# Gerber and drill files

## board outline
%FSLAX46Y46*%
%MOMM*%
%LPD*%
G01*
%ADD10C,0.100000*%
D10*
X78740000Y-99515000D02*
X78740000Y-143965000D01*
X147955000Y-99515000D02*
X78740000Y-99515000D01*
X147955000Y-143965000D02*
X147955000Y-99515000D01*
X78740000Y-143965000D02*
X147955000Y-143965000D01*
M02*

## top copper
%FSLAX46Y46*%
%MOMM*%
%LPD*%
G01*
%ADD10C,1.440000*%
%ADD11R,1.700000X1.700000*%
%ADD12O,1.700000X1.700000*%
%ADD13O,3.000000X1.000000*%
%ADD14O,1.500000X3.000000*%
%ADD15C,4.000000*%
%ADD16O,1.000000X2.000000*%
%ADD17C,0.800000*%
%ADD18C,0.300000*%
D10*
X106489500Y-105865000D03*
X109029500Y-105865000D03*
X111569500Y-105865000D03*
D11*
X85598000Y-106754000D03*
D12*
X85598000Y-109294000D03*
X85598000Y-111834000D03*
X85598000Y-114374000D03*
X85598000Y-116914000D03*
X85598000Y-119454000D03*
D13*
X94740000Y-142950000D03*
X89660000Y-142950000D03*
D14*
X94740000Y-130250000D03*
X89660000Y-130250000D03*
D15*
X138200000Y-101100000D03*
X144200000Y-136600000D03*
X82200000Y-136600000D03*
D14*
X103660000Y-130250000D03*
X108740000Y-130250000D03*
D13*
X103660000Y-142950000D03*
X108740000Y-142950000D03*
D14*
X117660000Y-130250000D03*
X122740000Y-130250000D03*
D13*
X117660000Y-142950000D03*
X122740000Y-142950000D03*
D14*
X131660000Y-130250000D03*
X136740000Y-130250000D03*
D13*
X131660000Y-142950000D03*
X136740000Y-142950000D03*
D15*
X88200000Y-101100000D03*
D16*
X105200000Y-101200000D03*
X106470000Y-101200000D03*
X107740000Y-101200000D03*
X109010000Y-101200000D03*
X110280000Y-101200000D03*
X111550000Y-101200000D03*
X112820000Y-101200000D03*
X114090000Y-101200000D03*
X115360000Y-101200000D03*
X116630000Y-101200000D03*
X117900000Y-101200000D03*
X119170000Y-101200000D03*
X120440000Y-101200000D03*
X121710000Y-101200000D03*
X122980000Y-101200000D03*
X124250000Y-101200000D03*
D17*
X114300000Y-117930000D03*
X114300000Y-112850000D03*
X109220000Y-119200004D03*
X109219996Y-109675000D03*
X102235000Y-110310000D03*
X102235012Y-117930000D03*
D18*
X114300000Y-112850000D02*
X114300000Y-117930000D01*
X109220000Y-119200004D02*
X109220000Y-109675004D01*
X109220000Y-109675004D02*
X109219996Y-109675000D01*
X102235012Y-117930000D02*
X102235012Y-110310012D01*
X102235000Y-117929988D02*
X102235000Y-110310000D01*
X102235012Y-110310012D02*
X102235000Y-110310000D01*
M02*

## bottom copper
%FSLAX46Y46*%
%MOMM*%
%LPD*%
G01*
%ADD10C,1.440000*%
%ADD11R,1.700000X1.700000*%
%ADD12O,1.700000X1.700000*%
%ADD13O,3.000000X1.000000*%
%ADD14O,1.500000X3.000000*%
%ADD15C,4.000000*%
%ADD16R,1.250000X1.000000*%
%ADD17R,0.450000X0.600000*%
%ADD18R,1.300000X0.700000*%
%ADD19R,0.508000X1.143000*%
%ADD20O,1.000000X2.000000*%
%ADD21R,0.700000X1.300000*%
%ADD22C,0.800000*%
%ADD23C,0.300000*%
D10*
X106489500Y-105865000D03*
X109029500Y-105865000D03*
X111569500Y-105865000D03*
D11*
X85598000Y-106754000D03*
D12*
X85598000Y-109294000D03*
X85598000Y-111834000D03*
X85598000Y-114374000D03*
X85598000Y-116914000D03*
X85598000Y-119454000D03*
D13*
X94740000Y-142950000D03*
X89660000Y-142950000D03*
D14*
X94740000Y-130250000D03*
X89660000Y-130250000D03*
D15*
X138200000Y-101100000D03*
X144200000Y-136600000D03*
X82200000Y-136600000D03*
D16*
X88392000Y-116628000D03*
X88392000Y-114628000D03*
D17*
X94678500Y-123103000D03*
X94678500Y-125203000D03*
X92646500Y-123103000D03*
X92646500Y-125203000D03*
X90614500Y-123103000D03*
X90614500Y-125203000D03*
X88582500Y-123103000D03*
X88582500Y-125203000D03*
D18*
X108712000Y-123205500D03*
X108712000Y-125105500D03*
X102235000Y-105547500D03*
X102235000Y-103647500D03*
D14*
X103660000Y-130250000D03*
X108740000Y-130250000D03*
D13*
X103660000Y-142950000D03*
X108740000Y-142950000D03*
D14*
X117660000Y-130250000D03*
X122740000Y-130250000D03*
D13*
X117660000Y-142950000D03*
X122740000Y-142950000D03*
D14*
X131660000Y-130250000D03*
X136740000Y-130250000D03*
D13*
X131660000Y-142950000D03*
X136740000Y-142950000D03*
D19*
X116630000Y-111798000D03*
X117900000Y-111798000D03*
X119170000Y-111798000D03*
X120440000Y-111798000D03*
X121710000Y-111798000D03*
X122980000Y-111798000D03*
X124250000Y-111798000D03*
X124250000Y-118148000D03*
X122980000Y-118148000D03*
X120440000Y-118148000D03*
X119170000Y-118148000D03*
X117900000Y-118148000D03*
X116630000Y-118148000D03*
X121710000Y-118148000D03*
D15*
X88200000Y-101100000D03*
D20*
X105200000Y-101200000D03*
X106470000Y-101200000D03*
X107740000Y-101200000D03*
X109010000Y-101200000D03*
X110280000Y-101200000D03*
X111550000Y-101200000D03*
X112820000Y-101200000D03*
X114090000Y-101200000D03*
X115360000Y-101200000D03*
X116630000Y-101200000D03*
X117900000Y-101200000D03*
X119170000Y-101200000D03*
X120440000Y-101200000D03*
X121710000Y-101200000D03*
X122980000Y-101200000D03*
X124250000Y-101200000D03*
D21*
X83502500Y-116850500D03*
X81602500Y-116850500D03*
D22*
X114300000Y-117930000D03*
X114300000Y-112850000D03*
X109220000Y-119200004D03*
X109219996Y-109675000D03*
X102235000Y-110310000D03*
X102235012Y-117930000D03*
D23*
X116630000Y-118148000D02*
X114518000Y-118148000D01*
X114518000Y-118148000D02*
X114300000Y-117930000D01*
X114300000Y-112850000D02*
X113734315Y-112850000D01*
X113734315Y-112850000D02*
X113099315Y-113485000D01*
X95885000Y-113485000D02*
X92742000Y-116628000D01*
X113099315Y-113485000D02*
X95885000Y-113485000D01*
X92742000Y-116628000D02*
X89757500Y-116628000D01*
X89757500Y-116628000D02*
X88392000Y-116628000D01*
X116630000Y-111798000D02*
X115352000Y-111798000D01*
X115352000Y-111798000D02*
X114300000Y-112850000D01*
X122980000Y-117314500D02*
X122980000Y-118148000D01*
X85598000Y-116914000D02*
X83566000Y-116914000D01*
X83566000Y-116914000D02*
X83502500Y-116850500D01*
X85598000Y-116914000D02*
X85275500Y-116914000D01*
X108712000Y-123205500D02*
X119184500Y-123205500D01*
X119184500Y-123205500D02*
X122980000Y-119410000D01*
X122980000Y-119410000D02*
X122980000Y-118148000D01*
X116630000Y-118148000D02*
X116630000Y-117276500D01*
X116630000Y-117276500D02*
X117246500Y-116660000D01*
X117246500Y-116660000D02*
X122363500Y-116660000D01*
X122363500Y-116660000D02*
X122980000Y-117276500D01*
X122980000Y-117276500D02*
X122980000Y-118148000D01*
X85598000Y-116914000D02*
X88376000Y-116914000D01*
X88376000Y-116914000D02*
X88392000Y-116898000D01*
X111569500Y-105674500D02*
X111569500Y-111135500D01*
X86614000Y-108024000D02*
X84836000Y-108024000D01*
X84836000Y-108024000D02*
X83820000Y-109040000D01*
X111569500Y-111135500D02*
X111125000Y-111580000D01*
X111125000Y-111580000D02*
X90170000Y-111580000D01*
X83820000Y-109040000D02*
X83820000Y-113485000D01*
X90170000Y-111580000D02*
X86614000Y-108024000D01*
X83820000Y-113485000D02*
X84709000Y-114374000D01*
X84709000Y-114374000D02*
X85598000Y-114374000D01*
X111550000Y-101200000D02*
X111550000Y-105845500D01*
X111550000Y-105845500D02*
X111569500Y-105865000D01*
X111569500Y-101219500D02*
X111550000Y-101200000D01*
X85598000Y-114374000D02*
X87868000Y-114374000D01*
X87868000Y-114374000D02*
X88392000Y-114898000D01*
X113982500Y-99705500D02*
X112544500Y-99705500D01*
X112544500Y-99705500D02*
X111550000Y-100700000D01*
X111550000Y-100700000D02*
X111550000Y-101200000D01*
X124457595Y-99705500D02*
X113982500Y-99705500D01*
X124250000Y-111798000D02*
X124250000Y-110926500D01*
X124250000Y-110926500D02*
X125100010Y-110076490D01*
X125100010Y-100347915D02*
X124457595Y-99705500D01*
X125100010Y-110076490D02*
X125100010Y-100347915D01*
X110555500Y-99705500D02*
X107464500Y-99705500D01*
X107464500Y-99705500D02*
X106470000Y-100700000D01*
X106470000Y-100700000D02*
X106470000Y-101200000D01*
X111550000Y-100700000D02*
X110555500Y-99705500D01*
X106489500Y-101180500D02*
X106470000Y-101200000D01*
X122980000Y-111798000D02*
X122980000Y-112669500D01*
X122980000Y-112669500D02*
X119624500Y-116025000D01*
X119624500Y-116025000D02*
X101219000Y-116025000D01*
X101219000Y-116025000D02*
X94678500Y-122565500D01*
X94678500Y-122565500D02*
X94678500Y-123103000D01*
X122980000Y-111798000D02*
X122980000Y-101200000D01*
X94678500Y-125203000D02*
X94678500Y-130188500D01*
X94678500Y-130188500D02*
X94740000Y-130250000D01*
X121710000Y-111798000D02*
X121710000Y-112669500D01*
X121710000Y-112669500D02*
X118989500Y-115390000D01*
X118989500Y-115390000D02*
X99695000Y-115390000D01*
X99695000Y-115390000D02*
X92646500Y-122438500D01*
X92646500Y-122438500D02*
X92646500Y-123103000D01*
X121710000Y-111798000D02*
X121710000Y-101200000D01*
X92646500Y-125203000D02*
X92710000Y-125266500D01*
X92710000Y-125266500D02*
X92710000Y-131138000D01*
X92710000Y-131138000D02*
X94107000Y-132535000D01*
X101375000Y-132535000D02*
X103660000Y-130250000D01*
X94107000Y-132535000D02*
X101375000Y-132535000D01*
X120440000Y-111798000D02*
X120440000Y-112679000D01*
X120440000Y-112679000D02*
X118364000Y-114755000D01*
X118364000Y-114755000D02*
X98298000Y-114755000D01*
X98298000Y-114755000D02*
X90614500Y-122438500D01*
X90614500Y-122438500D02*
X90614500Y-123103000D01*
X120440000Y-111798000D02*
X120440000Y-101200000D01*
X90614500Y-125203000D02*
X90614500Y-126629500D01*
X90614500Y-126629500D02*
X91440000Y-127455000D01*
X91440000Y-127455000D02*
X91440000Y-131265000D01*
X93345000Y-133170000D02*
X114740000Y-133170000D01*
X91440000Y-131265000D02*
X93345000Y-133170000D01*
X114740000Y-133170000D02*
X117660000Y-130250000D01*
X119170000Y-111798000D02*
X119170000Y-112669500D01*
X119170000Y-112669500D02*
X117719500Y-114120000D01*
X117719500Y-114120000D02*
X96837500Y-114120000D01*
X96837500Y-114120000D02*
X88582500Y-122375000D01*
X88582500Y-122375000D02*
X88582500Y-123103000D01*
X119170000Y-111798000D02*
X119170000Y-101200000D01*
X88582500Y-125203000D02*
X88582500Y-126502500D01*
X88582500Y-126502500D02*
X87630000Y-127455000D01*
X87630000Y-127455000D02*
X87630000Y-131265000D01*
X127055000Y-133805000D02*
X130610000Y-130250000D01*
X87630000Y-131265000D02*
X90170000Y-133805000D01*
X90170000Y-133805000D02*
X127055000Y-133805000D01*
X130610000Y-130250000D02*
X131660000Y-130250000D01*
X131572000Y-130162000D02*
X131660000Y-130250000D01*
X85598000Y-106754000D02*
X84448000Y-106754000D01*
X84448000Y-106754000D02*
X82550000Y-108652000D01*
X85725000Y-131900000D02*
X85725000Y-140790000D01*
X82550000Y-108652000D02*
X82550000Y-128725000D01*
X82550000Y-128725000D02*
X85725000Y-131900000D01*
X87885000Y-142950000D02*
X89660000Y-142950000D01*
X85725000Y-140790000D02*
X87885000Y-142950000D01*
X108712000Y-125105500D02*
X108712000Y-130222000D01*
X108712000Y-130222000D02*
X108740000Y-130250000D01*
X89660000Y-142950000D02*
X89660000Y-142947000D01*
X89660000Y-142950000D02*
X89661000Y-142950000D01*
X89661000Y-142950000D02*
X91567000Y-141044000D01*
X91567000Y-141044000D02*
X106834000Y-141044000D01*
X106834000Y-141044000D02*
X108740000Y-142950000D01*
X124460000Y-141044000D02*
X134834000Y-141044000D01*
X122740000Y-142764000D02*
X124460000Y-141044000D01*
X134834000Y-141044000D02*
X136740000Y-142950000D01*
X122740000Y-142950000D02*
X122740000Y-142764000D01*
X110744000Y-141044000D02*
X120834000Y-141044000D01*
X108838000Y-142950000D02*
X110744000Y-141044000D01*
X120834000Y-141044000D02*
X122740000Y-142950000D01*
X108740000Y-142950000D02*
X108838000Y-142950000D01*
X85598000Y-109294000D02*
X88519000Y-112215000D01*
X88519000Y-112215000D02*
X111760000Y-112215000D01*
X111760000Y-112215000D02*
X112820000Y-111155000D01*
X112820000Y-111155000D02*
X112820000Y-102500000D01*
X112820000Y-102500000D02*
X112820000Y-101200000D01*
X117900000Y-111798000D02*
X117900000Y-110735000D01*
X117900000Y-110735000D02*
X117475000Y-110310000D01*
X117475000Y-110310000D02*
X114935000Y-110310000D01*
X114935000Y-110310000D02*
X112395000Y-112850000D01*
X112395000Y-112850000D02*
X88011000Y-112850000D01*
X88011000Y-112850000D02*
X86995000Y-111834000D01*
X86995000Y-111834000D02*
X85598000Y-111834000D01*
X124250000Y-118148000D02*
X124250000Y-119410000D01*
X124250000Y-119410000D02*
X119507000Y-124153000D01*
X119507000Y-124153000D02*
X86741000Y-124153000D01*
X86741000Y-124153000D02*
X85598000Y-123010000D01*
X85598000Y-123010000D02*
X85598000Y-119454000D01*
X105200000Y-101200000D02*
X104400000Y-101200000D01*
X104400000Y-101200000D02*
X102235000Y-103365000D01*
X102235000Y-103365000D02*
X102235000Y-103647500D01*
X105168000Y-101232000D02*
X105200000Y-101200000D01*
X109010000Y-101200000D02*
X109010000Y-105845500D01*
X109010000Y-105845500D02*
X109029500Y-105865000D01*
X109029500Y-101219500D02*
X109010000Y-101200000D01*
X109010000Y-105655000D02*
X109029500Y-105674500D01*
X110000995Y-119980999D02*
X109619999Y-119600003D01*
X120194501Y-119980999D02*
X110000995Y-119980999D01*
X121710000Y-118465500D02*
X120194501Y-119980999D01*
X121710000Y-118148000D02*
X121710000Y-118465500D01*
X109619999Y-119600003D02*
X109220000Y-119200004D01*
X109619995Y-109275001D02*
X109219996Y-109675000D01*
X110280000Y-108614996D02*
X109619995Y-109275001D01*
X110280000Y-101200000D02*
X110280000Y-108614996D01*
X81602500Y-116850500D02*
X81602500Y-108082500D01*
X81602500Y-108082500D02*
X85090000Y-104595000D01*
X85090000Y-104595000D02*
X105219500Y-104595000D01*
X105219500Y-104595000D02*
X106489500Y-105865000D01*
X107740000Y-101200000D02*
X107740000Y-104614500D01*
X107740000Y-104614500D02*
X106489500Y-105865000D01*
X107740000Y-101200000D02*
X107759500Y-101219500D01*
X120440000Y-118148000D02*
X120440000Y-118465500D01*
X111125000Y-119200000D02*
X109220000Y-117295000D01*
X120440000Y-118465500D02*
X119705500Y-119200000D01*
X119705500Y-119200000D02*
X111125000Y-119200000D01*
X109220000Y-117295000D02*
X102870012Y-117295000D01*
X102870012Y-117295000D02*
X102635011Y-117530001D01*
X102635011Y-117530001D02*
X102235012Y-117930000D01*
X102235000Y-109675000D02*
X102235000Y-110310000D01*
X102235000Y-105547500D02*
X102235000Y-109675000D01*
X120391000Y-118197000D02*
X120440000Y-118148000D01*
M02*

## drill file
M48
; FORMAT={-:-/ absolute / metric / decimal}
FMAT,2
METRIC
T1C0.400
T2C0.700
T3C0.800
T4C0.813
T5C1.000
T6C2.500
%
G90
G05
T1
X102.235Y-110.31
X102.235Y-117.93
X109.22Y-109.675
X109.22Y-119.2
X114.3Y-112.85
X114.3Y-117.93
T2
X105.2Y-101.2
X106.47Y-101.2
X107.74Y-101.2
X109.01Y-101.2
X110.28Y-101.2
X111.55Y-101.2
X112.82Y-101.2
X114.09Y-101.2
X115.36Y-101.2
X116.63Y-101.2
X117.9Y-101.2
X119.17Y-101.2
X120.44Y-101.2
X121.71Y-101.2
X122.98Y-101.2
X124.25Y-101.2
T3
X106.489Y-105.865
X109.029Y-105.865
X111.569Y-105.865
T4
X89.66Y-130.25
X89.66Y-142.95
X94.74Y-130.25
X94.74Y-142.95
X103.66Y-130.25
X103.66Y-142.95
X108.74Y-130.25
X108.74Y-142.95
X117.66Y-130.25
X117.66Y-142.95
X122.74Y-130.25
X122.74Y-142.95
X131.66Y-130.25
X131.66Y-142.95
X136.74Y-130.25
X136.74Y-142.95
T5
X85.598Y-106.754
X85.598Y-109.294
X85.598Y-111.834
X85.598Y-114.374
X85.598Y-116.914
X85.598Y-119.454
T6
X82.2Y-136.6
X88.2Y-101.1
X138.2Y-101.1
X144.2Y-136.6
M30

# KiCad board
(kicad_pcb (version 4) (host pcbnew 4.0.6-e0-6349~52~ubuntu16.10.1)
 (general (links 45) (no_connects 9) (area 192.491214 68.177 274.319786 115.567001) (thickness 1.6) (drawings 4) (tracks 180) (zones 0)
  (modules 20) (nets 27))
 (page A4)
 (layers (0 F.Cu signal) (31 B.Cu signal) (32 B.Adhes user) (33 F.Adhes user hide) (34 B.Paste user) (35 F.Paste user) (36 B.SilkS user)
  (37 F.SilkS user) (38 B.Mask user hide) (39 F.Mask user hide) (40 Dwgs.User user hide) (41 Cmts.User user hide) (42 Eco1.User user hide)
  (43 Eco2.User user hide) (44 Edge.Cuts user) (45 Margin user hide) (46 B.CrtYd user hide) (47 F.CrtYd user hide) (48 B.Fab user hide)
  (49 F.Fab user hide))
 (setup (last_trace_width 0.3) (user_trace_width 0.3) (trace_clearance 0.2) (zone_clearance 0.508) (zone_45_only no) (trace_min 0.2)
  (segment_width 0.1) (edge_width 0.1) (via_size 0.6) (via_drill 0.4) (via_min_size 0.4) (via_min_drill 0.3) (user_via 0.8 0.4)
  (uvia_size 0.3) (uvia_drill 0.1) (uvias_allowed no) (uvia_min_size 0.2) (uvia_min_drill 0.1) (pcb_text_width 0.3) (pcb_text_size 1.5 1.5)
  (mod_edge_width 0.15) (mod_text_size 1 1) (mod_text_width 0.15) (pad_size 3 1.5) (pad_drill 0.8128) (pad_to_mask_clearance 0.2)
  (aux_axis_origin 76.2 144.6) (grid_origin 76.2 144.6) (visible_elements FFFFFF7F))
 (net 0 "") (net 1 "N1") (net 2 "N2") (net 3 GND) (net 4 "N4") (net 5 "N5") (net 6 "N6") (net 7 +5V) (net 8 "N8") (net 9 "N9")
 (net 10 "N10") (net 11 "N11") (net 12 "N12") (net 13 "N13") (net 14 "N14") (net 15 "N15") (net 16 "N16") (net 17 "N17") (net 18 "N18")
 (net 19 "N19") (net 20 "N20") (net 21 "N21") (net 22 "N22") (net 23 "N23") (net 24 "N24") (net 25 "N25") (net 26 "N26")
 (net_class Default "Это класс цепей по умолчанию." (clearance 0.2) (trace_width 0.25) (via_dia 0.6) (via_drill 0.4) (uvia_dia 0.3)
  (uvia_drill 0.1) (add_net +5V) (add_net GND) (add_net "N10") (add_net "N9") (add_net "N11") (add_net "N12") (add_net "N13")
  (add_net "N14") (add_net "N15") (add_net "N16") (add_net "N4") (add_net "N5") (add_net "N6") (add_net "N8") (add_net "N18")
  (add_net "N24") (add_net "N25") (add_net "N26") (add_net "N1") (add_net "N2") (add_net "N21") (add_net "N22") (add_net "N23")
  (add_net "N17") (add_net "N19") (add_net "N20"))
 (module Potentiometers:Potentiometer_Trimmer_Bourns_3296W (layer B.Cu) (at 106.4895 105.865 180)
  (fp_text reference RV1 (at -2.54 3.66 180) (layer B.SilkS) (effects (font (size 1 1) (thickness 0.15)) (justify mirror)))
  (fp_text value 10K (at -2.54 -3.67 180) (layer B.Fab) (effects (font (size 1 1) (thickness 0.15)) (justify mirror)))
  (pad 1 thru_hole circle (at 0 0 180) (size 1.44 1.44) (drill 0.8) (layers *.Cu *.Mask) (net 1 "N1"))
  (pad 2 thru_hole circle (at -2.54 0 180) (size 1.44 1.44) (drill 0.8) (layers *.Cu *.Mask) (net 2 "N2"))
  (pad 3 thru_hole circle (at -5.08 0 180) (size 1.44 1.44) (drill 0.8) (layers *.Cu *.Mask) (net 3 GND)))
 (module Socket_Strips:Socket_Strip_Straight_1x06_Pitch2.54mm (layer B.Cu) (at 85.598 106.754 180)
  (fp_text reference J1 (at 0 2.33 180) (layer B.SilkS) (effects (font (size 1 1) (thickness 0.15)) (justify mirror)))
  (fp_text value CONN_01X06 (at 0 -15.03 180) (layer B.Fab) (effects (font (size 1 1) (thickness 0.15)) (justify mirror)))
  (pad 1 thru_hole rect (at 0 0 180) (size 1.7 1.7) (drill 1) (layers *.Cu *.Mask) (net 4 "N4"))
  (pad 2 thru_hole oval (at 0 -2.54 180) (size 1.7 1.7) (drill 1) (layers *.Cu *.Mask) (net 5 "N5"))
  (pad 3 thru_hole oval (at 0 -5.08 180) (size 1.7 1.7) (drill 1) (layers *.Cu *.Mask) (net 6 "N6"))
  (pad 4 thru_hole oval (at 0 -7.62 180) (size 1.7 1.7) (drill 1) (layers *.Cu *.Mask) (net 3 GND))
  (pad 5 thru_hole oval (at 0 -10.16 180) (size 1.7 1.7) (drill 1) (layers *.Cu *.Mask) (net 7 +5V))
  (pad 6 thru_hole oval (at 0 -12.7 180) (size 1.7 1.7) (drill 1) (layers *.Cu *.Mask) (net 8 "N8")))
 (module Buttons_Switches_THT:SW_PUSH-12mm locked (layer F.Cu) (at 92.2 136.6 270)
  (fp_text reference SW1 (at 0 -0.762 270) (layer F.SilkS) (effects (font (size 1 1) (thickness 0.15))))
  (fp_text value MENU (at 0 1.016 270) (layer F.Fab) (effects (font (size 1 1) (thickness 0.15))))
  (pad 1 thru_hole oval (at 6.35 -2.54) (size 3 1) (drill 0.8128) (layers *.Cu *.Mask) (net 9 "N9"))
  (pad 2 thru_hole oval (at 6.35 2.54) (size 3 1) (drill 0.8128) (layers *.Cu *.Mask) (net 4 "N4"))
  (pad 1 thru_hole oval (at -6.35 -2.54 270) (size 3 1.5) (drill 0.8128) (layers *.Cu *.Mask) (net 9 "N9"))
  (pad 2 thru_hole oval (at -6.35 2.54 270) (size 3 1.5) (drill 0.8128) (layers *.Cu *.Mask) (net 4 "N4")))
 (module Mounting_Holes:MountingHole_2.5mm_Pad (layer F.Cu) (at 138.2 101.1)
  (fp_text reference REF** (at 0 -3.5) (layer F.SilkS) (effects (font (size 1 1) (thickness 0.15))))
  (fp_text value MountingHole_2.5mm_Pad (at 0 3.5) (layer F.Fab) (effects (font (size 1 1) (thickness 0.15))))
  (pad 1 thru_hole circle (at 0 0) (size 4 4) (drill 2.5) (layers *.Cu *.Mask)))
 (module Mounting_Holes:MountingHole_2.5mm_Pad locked (layer F.Cu) (at 144.2 136.6)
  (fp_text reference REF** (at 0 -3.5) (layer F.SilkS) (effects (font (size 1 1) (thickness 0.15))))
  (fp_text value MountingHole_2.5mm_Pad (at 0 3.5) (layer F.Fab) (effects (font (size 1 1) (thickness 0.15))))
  (pad 1 thru_hole circle (at 0 0) (size 4 4) (drill 2.5) (layers *.Cu *.Mask)))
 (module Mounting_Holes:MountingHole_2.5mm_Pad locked (layer F.Cu) (at 82.2 136.6)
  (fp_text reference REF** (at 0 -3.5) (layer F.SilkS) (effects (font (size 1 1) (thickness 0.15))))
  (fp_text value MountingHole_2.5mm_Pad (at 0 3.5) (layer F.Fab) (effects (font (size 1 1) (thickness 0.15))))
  (pad 1 thru_hole circle (at 0 0) (size 4 4) (drill 2.5) (layers *.Cu *.Mask)))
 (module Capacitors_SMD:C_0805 (layer B.Cu) (at 88.392 115.628 90)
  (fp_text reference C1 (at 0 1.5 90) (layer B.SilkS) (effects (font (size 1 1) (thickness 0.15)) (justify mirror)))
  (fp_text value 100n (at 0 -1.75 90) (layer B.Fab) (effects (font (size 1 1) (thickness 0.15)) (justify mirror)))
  (pad 1 smd rect (at -1 0 90) (size 1 1.25) (layers B.Cu B.Paste B.Mask) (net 7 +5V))
  (pad 2 smd rect (at 1 0 90) (size 1 1.25) (layers B.Cu B.Paste B.Mask) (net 3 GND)))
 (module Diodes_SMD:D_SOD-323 (layer B.Cu) (at 94.6785 124.153 270)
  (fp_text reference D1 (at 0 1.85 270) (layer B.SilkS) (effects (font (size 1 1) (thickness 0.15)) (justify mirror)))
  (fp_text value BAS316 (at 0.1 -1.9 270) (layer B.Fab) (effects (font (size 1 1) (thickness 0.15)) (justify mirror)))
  (pad 1 smd rect (at -1.05 0 270) (size 0.6 0.45) (layers B.Cu B.Paste B.Mask) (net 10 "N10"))
  (pad 2 smd rect (at 1.05 0 270) (size 0.6 0.45) (layers B.Cu B.Paste B.Mask) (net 9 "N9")))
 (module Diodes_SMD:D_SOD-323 (layer B.Cu) (at 92.6465 124.153 270)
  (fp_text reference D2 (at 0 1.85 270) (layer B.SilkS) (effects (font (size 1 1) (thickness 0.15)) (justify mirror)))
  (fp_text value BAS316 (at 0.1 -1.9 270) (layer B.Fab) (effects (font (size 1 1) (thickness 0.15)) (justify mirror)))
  (pad 1 smd rect (at -1.05 0 270) (size 0.6 0.45) (layers B.Cu B.Paste B.Mask) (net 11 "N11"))
  (pad 2 smd rect (at 1.05 0 270) (size 0.6 0.45) (layers B.Cu B.Paste B.Mask) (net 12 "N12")))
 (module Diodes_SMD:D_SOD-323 (layer B.Cu) (at 90.6145 124.153 270)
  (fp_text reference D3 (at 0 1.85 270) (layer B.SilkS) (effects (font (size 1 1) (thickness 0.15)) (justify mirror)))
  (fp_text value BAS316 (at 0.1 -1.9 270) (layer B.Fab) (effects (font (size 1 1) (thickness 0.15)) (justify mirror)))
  (pad 1 smd rect (at -1.05 0 270) (size 0.6 0.45) (layers B.Cu B.Paste B.Mask) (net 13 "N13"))
  (pad 2 smd rect (at 1.05 0 270) (size 0.6 0.45) (layers B.Cu B.Paste B.Mask) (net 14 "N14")))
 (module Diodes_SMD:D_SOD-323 (layer B.Cu) (at 88.5825 124.153 270)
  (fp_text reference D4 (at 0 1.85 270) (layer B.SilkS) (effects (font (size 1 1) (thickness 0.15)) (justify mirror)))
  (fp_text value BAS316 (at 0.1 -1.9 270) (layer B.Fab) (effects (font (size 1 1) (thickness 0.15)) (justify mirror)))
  (pad 1 smd rect (at -1.05 0 270) (size 0.6 0.45) (layers B.Cu B.Paste B.Mask) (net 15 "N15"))
  (pad 2 smd rect (at 1.05 0 270) (size 0.6 0.45) (layers B.Cu B.Paste B.Mask) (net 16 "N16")))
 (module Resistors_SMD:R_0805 (layer B.Cu) (at 108.712 124.1555 270)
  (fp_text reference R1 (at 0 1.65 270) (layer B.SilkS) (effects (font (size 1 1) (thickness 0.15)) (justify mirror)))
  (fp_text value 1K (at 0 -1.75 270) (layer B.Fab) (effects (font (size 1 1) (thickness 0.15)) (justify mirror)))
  (pad 1 smd rect (at -0.95 0 270) (size 0.7 1.3) (layers B.Cu B.Paste B.Mask) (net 7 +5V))
  (pad 2 smd rect (at 0.95 0 270) (size 0.7 1.3) (layers B.Cu B.Paste B.Mask) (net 4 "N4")))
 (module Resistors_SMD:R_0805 (layer B.Cu) (at 102.235 104.5975 90)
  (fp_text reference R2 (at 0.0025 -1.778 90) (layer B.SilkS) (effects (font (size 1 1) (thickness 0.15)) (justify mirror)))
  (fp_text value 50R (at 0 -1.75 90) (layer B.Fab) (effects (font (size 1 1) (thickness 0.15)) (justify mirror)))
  (pad 1 smd rect (at -0.95 0 90) (size 0.7 1.3) (layers B.Cu B.Paste B.Mask) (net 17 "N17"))
  (pad 2 smd rect (at 0.95 0 90) (size 0.7 1.3) (layers B.Cu B.Paste B.Mask) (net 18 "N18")))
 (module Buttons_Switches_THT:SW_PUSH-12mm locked (layer F.Cu) (at 106.2 136.6 90)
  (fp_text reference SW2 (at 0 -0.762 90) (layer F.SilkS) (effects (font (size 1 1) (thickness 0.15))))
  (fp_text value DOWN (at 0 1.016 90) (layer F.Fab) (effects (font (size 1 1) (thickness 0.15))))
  (pad 1 thru_hole oval (at 6.35 -2.54 90) (size 3 1.5) (drill 0.8128) (layers *.Cu *.Mask) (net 12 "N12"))
  (pad 2 thru_hole oval (at 6.35 2.54 90) (size 3 1.5) (drill 0.8128) (layers *.Cu *.Mask) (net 4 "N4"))
  (pad 1 thru_hole oval (at -6.35 -2.54 180) (size 3 1) (drill 0.8128) (layers *.Cu *.Mask) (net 12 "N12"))
  (pad 2 thru_hole oval (at -6.35 2.54 180) (size 3 1) (drill 0.8128) (layers *.Cu *.Mask) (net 4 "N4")))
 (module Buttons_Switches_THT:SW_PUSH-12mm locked (layer F.Cu) (at 120.2 136.6 90)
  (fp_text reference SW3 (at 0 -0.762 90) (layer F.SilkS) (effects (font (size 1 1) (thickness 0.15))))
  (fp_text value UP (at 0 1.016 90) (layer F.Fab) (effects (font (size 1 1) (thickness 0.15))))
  (pad 1 thru_hole oval (at 6.35 -2.54 90) (size 3 1.5) (drill 0.8128) (layers *.Cu *.Mask) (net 14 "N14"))
  (pad 2 thru_hole oval (at 6.35 2.54 90) (size 3 1.5) (drill 0.8128) (layers *.Cu *.Mask) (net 4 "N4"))
  (pad 1 thru_hole oval (at -6.35 -2.54 180) (size 3 1) (drill 0.8128) (layers *.Cu *.Mask) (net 14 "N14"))
  (pad 2 thru_hole oval (at -6.35 2.54 180) (size 3 1) (drill 0.8128) (layers *.Cu *.Mask) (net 4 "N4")))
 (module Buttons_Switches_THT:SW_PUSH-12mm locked (layer F.Cu) (at 134.2 136.6 90)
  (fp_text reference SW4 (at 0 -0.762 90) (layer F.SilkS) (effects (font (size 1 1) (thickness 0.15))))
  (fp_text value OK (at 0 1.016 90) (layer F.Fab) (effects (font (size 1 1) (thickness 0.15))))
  (pad 1 thru_hole oval (at 6.35 -2.54 90) (size 3 1.5) (drill 0.8128) (layers *.Cu *.Mask) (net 16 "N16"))
  (pad 2 thru_hole oval (at 6.35 2.54 90) (size 3 1.5) (drill 0.8128) (layers *.Cu *.Mask) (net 4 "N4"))
  (pad 1 thru_hole oval (at -6.35 -2.54 180) (size 3 1) (drill 0.8128) (layers *.Cu *.Mask) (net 16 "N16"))
  (pad 2 thru_hole oval (at -6.35 2.54 180) (size 3 1) (drill 0.8128) (layers *.Cu *.Mask) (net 4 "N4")))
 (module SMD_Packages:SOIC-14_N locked (layer B.Cu) (at 120.44 115.1)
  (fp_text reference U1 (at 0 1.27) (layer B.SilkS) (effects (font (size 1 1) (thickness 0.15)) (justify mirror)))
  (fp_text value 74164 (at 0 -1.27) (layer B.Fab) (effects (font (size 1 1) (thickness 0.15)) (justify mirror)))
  (pad 1 smd rect (at -3.81 -3.302) (size 0.508 1.143) (layers B.Cu B.Paste B.Mask) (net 7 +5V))
  (pad 2 smd rect (at -2.54 -3.302) (size 0.508 1.143) (layers B.Cu B.Paste B.Mask) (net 6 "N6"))
  (pad 3 smd rect (at -1.27 -3.302) (size 0.508 1.143) (layers B.Cu B.Paste B.Mask) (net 15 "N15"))
  (pad 4 smd rect (at 0 -3.302) (size 0.508 1.143) (layers B.Cu B.Paste B.Mask) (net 13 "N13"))
  (pad 5 smd rect (at 1.27 -3.302) (size 0.508 1.143) (layers B.Cu B.Paste B.Mask) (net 11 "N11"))
  (pad 6 smd rect (at 2.54 -3.302) (size 0.508 1.143) (layers B.Cu B.Paste B.Mask) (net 10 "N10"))
  (pad 7 smd rect (at 3.81 -3.302) (size 0.508 1.143) (layers B.Cu B.Paste B.Mask) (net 3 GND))
  (pad 8 smd rect (at 3.81 3.048) (size 0.508 1.143) (layers B.Cu B.Paste B.Mask) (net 8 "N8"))
  (pad 9 smd rect (at 2.54 3.048) (size 0.508 1.143) (layers B.Cu B.Paste B.Mask) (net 7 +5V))
  (pad 11 smd rect (at 0 3.048) (size 0.508 1.143) (layers B.Cu B.Paste B.Mask) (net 17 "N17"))
  (pad 12 smd rect (at -1.27 3.048) (size 0.508 1.143) (layers B.Cu B.Paste B.Mask) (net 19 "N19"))
  (pad 13 smd rect (at -2.54 3.048) (size 0.508 1.143) (layers B.Cu B.Paste B.Mask) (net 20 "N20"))
  (pad 14 smd rect (at -3.81 3.048) (size 0.508 1.143) (layers B.Cu B.Paste B.Mask) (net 7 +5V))
  (pad 10 smd rect (at 1.27 3.048) (size 0.508 1.143) (layers B.Cu B.Paste B.Mask) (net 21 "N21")))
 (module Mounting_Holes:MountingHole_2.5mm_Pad (layer F.Cu) (at 88.2 101.1)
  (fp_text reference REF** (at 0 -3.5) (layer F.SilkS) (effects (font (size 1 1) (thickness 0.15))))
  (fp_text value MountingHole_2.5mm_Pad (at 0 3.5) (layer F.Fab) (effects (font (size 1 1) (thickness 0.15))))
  (pad 1 thru_hole circle (at 0 0) (size 4 4) (drill 2.5) (layers *.Cu *.Mask)))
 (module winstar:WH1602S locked (layer F.Cu) (at 113.2 115.1)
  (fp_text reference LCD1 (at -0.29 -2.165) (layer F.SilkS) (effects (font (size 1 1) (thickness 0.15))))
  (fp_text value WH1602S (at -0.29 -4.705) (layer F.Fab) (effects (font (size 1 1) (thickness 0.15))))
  (pad 1 thru_hole oval (at -8 -13.9) (size 1 2) (drill 0.7) (layers *.Cu *.Mask) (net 18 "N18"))
  (pad 2 thru_hole oval (at -6.73 -13.9) (size 1 2) (drill 0.7) (layers *.Cu *.Mask) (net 3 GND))
  (pad 3 thru_hole oval (at -5.46 -13.9) (size 1 2) (drill 0.7) (layers *.Cu *.Mask) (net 1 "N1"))
  (pad 4 thru_hole oval (at -4.19 -13.9) (size 1 2) (drill 0.7) (layers *.Cu *.Mask) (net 2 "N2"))
  (pad 5 thru_hole oval (at -2.92 -13.9) (size 1 2) (drill 0.7) (layers *.Cu *.Mask) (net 21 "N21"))
  (pad 6 thru_hole oval (at -1.65 -13.9) (size 1 2) (drill 0.7) (layers *.Cu *.Mask) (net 3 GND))
  (pad 7 thru_hole oval (at -0.38 -13.9) (size 1 2) (drill 0.7) (layers *.Cu *.Mask) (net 5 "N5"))
  (pad 8 thru_hole oval (at 0.89 -13.9) (size 1 2) (drill 0.7) (layers *.Cu *.Mask) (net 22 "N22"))
  (pad 9 thru_hole oval (at 2.16 -13.9) (size 1 2) (drill 0.7) (layers *.Cu *.Mask) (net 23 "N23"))
  (pad 10 thru_hole oval (at 3.43 -13.9) (size 1 2) (drill 0.7) (layers *.Cu *.Mask) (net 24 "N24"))
  (pad 11 thru_hole oval (at 4.7 -13.9) (size 1 2) (drill 0.7) (layers *.Cu *.Mask) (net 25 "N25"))
  (pad 12 thru_hole oval (at 5.97 -13.9) (size 1 2) (drill 0.7) (layers *.Cu *.Mask) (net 15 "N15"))
  (pad 13 thru_hole oval (at 7.24 -13.9) (size 1 2) (drill 0.7) (layers *.Cu *.Mask) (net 13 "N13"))
  (pad 14 thru_hole oval (at 8.51 -13.9) (size 1 2) (drill 0.7) (layers *.Cu *.Mask) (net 11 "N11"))
  (pad 15 thru_hole oval (at 9.78 -13.9) (size 1 2) (drill 0.7) (layers *.Cu *.Mask) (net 10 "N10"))
  (pad 16 thru_hole oval (at 11.05 -13.9) (size 1 2) (drill 0.7) (layers *.Cu *.Mask) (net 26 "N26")))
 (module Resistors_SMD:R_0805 (layer B.Cu) (at 82.5525 116.8505 180)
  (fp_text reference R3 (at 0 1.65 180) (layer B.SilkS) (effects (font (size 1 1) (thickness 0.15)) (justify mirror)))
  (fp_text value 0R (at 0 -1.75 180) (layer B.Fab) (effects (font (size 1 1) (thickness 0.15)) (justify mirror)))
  (pad 1 smd rect (at -0.95 0 180) (size 0.7 1.3) (layers B.Cu B.Paste B.Mask) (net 7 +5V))
  (pad 2 smd rect (at 0.95 0 180) (size 0.7 1.3) (layers B.Cu B.Paste B.Mask) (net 1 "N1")))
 (gr_line (start 78.74 99.515) (end 78.74 143.965) (layer Edge.Cuts) (width 0.1))
 (gr_line (start 147.955 99.515) (end 78.74 99.515) (layer Edge.Cuts) (width 0.1))
 (gr_line (start 147.955 143.965) (end 147.955 99.515) (layer Edge.Cuts) (width 0.1))
 (gr_line (start 78.74 143.965) (end 147.955 143.965) (layer Edge.Cuts) (width 0.1))
 (segment (start 116.63 118.148) (end 114.518 118.148) (width 0.3) (layer B.Cu) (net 7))
 (segment (start 114.3 112.85) (end 114.3 117.93) (width 0.3) (layer F.Cu) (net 7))
 (via (at 114.3 117.93) (size 0.8) (drill 0.4) (layers F.Cu B.Cu) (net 7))
 (segment (start 114.518 118.148) (end 114.3 117.93) (width 0.3) (layer B.Cu) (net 7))
 (segment (start 114.3 112.85) (end 113.734315 112.85) (width 0.3) (layer B.Cu) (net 7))
 (segment (start 113.734315 112.85) (end 113.099315 113.485) (width 0.3) (layer B.Cu) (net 7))
 (segment (start 95.885 113.485) (end 92.742 116.628) (width 0.3) (layer B.Cu) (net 7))
 (segment (start 113.099315 113.485) (end 95.885 113.485) (width 0.3) (layer B.Cu) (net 7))
 (segment (start 92.742 116.628) (end 89.7575 116.628) (width 0.3) (layer B.Cu) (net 7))
 (segment (start 89.7575 116.628) (end 88.392 116.628) (width 0.3) (layer B.Cu) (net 7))
 (segment (start 116.63 111.798) (end 115.352 111.798) (width 0.3) (layer B.Cu) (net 7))
 (via (at 114.3 112.85) (size 0.8) (drill 0.4) (layers F.Cu B.Cu) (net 7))
 (segment (start 115.352 111.798) (end 114.3 112.85) (width 0.3) (layer B.Cu) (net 7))
 (segment (start 122.98 117.3145) (end 122.98 118.148) (width 0.3) (layer B.Cu) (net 7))
 (segment (start 85.598 116.914) (end 83.566 116.914) (width 0.3) (layer B.Cu) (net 7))
 (segment (start 83.566 116.914) (end 83.5025 116.8505) (width 0.3) (layer B.Cu) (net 7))
 (segment (start 85.598 116.914) (end 85.2755 116.914) (width 0.3) (layer B.Cu) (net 7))
 (segment (start 108.712 123.2055) (end 119.1845 123.2055) (width 0.3) (layer B.Cu) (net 7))
 (segment (start 119.1845 123.2055) (end 122.98 119.41) (width 0.3) (layer B.Cu) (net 7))
 (segment (start 122.98 119.41) (end 122.98 118.148) (width 0.3) (layer B.Cu) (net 7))
 (segment (start 116.63 118.148) (end 116.63 117.2765) (width 0.3) (layer B.Cu) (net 7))
 (segment (start 116.63 117.2765) (end 117.2465 116.66) (width 0.3) (layer B.Cu) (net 7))
 (segment (start 117.2465 116.66) (end 122.3635 116.66) (width 0.3) (layer B.Cu) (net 7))
 (segment (start 122.3635 116.66) (end 122.98 117.2765) (width 0.3) (layer B.Cu) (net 7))
 (segment (start 122.98 117.2765) (end 122.98 118.148) (width 0.3) (layer B.Cu) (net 7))
 (segment (start 85.598 116.914) (end 88.376 116.914) (width 0.3) (layer B.Cu) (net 7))
 (segment (start 88.376 116.914) (end 88.392 116.898) (width 0.3) (layer B.Cu) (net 7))
 (segment (start 111.5695 105.6745) (end 111.5695 111.1355) (width 0.3) (layer B.Cu) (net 3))
 (segment (start 86.614 108.024) (end 84.836 108.024) (width 0.3) (layer B.Cu) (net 3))
 (segment (start 84.836 108.024) (end 83.82 109.04) (width 0.3) (layer B.Cu) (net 3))
 (segment (start 111.5695 111.1355) (end 111.125 111.58) (width 0.3) (layer B.Cu) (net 3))
 (segment (start 111.125 111.58) (end 90.17 111.58) (width 0.3) (layer B.Cu) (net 3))
 (segment (start 83.82 109.04) (end 83.82 113.485) (width 0.3) (layer B.Cu) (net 3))
 (segment (start 90.17 111.58) (end 86.614 108.024) (width 0.3) (layer B.Cu) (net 3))
 (segment (start 83.82 113.485) (end 84.709 114.374) (width 0.3) (layer B.Cu) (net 3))
 (segment (start 84.709 114.374) (end 85.598 114.374) (width 0.3) (layer B.Cu) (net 3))
 (segment (start 111.55 101.2) (end 111.55 105.8455) (width 0.3) (layer B.Cu) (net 3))
 (segment (start 111.55 105.8455) (end 111.5695 105.865) (width 0.3) (layer B.Cu) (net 3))
 (segment (start 111.5695 101.2195) (end 111.55 101.2) (width 0.3) (layer B.Cu) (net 3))
 (segment (start 85.598 114.374) (end 87.868 114.374) (width 0.3) (layer B.Cu) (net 3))
 (segment (start 87.868 114.374) (end 88.392 114.898) (width 0.3) (layer B.Cu) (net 3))
 (segment (start 113.9825 99.7055) (end 112.5445 99.7055) (width 0.3) (layer B.Cu) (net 3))
 (segment (start 112.5445 99.7055) (end 111.55 100.7) (width 0.3) (layer B.Cu) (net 3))
 (segment (start 111.55 100.7) (end 111.55 101.2) (width 0.3) (layer B.Cu) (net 3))
 (segment (start 124.457595 99.7055) (end 113.9825 99.7055) (width 0.3) (layer B.Cu) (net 3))
 (segment (start 124.25 111.798) (end 124.25 110.9265) (width 0.3) (layer B.Cu) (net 3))
 (segment (start 124.25 110.9265) (end 125.10001 110.07649) (width 0.3) (layer B.Cu) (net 3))
 (segment (start 125.10001 100.347915) (end 124.457595 99.7055) (width 0.3) (layer B.Cu) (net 3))
 (segment (start 125.10001 110.07649) (end 125.10001 100.347915) (width 0.3) (layer B.Cu) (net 3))
 (segment (start 110.5555 99.7055) (end 107.4645 99.7055) (width 0.3) (layer B.Cu) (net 3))
 (segment (start 107.4645 99.7055) (end 106.47 100.7) (width 0.3) (layer B.Cu) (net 3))
 (segment (start 106.47 100.7) (end 106.47 101.2) (width 0.3) (layer B.Cu) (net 3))
 (segment (start 111.55 100.7) (end 110.5555 99.7055) (width 0.3) (layer B.Cu) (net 3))
 (segment (start 106.4895 101.1805) (end 106.47 101.2) (width 0.3) (layer B.Cu) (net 3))
 (segment (start 122.98 111.798) (end 122.98 112.6695) (width 0.3) (layer B.Cu) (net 10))
 (segment (start 122.98 112.6695) (end 119.6245 116.025) (width 0.3) (layer B.Cu) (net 10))
 (segment (start 119.6245 116.025) (end 101.219 116.025) (width 0.3) (layer B.Cu) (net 10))
 (segment (start 101.219 116.025) (end 94.6785 122.5655) (width 0.3) (layer B.Cu) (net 10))
 (segment (start 94.6785 122.5655) (end 94.6785 123.103) (width 0.3) (layer B.Cu) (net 10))
 (segment (start 122.98 111.798) (end 122.98 101.2) (width 0.3) (layer B.Cu) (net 10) (status 10))
 (segment (start 94.6785 125.203) (end 94.6785 130.1885) (width 0.3) (layer B.Cu) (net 9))
 (segment (start 94.6785 130.1885) (end 94.74 130.25) (width 0.3) (layer B.Cu) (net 9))
 (segment (start 121.71 111.798) (end 121.71 112.6695) (width 0.3) (layer B.Cu) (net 11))
 (segment (start 121.71 112.6695) (end 118.9895 115.39) (width 0.3) (layer B.Cu) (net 11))
 (segment (start 118.9895 115.39) (end 99.695 115.39) (width 0.3) (layer B.Cu) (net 11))
 (segment (start 99.695 115.39) (end 92.6465 122.4385) (width 0.3) (layer B.Cu) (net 11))
 (segment (start 92.6465 122.4385) (end 92.6465 123.103) (width 0.3) (layer B.Cu) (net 11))
 (segment (start 121.71 111.798) (end 121.71 101.2) (width 0.3) (layer B.Cu) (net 11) (status 10))
 (segment (start 92.6465 125.203) (end 92.71 125.2665) (width 0.3) (layer B.Cu) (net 12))
 (segment (start 92.71 125.2665) (end 92.71 131.138) (width 0.3) (layer B.Cu) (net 12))
 (segment (start 92.71 131.138) (end 94.107 132.535) (width 0.3) (layer B.Cu) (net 12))
 (segment (start 101.375 132.535) (end 103.66 130.25) (width 0.3) (layer B.Cu) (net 12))
 (segment (start 94.107 132.535) (end 101.375 132.535) (width 0.3) (layer B.Cu) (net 12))
 (segment (start 120.44 111.798) (end 120.44 112.679) (width 0.3) (layer B.Cu) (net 13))
 (segment (start 120.44 112.679) (end 118.364 114.755) (width 0.3) (layer B.Cu) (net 13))
 (segment (start 118.364 114.755) (end 98.298 114.755) (width 0.3) (layer B.Cu) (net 13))
 (segment (start 98.298 114.755) (end 90.6145 122.4385) (width 0.3) (layer B.Cu) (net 13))
 (segment (start 90.6145 122.4385) (end 90.6145 123.103) (width 0.3) (layer B.Cu) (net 13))
 (segment (start 120.44 111.798) (end 120.44 101.2) (width 0.3) (layer B.Cu) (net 13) (status 10))
 (segment (start 90.6145 125.203) (end 90.6145 126.6295) (width 0.3) (layer B.Cu) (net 14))
 (segment (start 90.6145 126.6295) (end 91.44 127.455) (width 0.3) (layer B.Cu) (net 14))
 (segment (start 91.44 127.455) (end 91.44 131.265) (width 0.3) (layer B.Cu) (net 14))
 (segment (start 93.345 133.17) (end 114.74 133.17) (width 0.3) (layer B.Cu) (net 14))
 (segment (start 91.44 131.265) (end 93.345 133.17) (width 0.3) (layer B.Cu) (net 14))
 (segment (start 114.74 133.17) (end 117.66 130.25) (width 0.3) (layer B.Cu) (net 14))
 (segment (start 119.17 111.798) (end 119.17 112.6695) (width 0.3) (layer B.Cu) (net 15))
 (segment (start 119.17 112.6695) (end 117.7195 114.12) (width 0.3) (layer B.Cu) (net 15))
 (segment (start 117.7195 114.12) (end 96.8375 114.12) (width 0.3) (layer B.Cu) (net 15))
 (segment (start 96.8375 114.12) (end 88.5825 122.375) (width 0.3) (layer B.Cu) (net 15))
 (segment (start 88.5825 122.375) (end 88.5825 123.103) (width 0.3) (layer B.Cu) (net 15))
 (segment (start 119.17 111.798) (end 119.17 101.2) (width 0.3) (layer B.Cu) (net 15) (status 10))
 (segment (start 88.5825 125.203) (end 88.5825 126.5025) (width 0.3) (layer B.Cu) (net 16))
 (segment (start 88.5825 126.5025) (end 87.63 127.455) (width 0.3) (layer B.Cu) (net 16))
 (segment (start 87.63 127.455) (end 87.63 131.265) (width 0.3) (layer B.Cu) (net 16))
 (segment (start 127.055 133.805) (end 130.61 130.25) (width 0.3) (layer B.Cu) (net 16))
 (segment (start 87.63 131.265) (end 90.17 133.805) (width 0.3) (layer B.Cu) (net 16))
 (segment (start 90.17 133.805) (end 127.055 133.805) (width 0.3) (layer B.Cu) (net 16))
 (segment (start 130.61 130.25) (end 131.66 130.25) (width 0.3) (layer B.Cu) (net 16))
 (segment (start 131.572 130.162) (end 131.66 130.25) (width 0.3) (layer B.Cu) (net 16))
 (segment (start 85.598 106.754) (end 84.448 106.754) (width 0.3) (layer B.Cu) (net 4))
 (segment (start 84.448 106.754) (end 82.55 108.652) (width 0.3) (layer B.Cu) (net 4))
 (segment (start 85.725 131.9) (end 85.725 140.79) (width 0.3) (layer B.Cu) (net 4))
 (segment (start 82.55 108.652) (end 82.55 128.725) (width 0.3) (layer B.Cu) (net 4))
 (segment (start 82.55 128.725) (end 85.725 131.9) (width 0.3) (layer B.Cu) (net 4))
 (segment (start 87.885 142.95) (end 89.66 142.95) (width 0.3) (layer B.Cu) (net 4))
 (segment (start 85.725 140.79) (end 87.885 142.95) (width 0.3) (layer B.Cu) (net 4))
 (segment (start 108.712 125.1055) (end 108.712 130.222) (width 0.3) (layer B.Cu) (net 4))
 (segment (start 108.712 130.222) (end 108.74 130.25) (width 0.3) (layer B.Cu) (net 4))
 (segment (start 89.66 142.95) (end 89.66 142.947) (width 0.3) (layer B.Cu) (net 4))
 (segment (start 89.66 142.95) (end 89.661 142.95) (width 0.3) (layer B.Cu) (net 4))
 (segment (start 89.661 142.95) (end 91.567 141.044) (width 0.3) (layer B.Cu) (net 4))
 (segment (start 91.567 141.044) (end 106.834 141.044) (width 0.3) (layer B.Cu) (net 4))
 (segment (start 106.834 141.044) (end 108.74 142.95) (width 0.3) (layer B.Cu) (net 4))
 (segment (start 124.46 141.044) (end 134.834 141.044) (width 0.3) (layer B.Cu) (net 4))
 (segment (start 122.74 142.764) (end 124.46 141.044) (width 0.3) (layer B.Cu) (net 4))
 (segment (start 134.834 141.044) (end 136.74 142.95) (width 0.3) (layer B.Cu) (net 4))
 (segment (start 122.74 142.95) (end 122.74 142.764) (width 0.3) (layer B.Cu) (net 4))
 (segment (start 110.744 141.044) (end 120.834 141.044) (width 0.3) (layer B.Cu) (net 4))
 (segment (start 108.838 142.95) (end 110.744 141.044) (width 0.3) (layer B.Cu) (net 4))
 (segment (start 120.834 141.044) (end 122.74 142.95) (width 0.3) (layer B.Cu) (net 4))
 (segment (start 108.74 142.95) (end 108.838 142.95) (width 0.3) (layer B.Cu) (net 4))
 (segment (start 85.598 109.294) (end 88.519 112.215) (width 0.3) (layer B.Cu) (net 5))
 (segment (start 88.519 112.215) (end 111.76 112.215) (width 0.3) (layer B.Cu) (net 5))
 (segment (start 111.76 112.215) (end 112.82 111.155) (width 0.3) (layer B.Cu) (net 5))
 (segment (start 112.82 111.155) (end 112.82 102.5) (width 0.3) (layer B.Cu) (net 5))
 (segment (start 112.82 102.5) (end 112.82 101.2) (width 0.3) (layer B.Cu) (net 5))
 (segment (start 117.9 111.798) (end 117.9 110.735) (width 0.3) (layer B.Cu) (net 6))
 (segment (start 117.9 110.735) (end 117.475 110.31) (width 0.3) (layer B.Cu) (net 6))
 (segment (start 117.475 110.31) (end 114.935 110.31) (width 0.3) (layer B.Cu) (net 6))
 (segment (start 114.935 110.31) (end 112.395 112.85) (width 0.3) (layer B.Cu) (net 6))
 (segment (start 112.395 112.85) (end 88.011 112.85) (width 0.3) (layer B.Cu) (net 6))
 (segment (start 88.011 112.85) (end 86.995 111.834) (width 0.3) (layer B.Cu) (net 6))
 (segment (start 86.995 111.834) (end 85.598 111.834) (width 0.3) (layer B.Cu) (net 6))
 (segment (start 124.25 118.148) (end 124.25 119.41) (width 0.3) (layer B.Cu) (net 8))
 (segment (start 124.25 119.41) (end 119.507 124.153) (width 0.3) (layer B.Cu) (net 8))
 (segment (start 119.507 124.153) (end 86.741 124.153) (width 0.3) (layer B.Cu) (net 8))
 (segment (start 86.741 124.153) (end 85.598 123.01) (width 0.3) (layer B.Cu) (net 8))
 (segment (start 85.598 123.01) (end 85.598 119.454) (width 0.3) (layer B.Cu) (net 8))
 (segment (start 105.2 101.2) (end 104.4 101.2) (width 0.3) (layer B.Cu) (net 18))
 (segment (start 104.4 101.2) (end 102.235 103.365) (width 0.3) (layer B.Cu) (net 18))
 (segment (start 102.235 103.365) (end 102.235 103.6475) (width 0.3) (layer B.Cu) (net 18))
 (segment (start 105.168 101.232) (end 105.2 101.2) (width 0.3) (layer B.Cu) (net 18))
 (segment (start 109.01 101.2) (end 109.01 105.8455) (width 0.3) (layer B.Cu) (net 2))
 (segment (start 109.01 105.8455) (end 109.0295 105.865) (width 0.3) (layer B.Cu) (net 2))
 (segment (start 109.0295 101.2195) (end 109.01 101.2) (width 0.3) (layer B.Cu) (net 2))
 (segment (start 109.01 105.655) (end 109.0295 105.6745) (width 0.3) (layer B.Cu) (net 2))
 (segment (start 109.22 119.200004) (end 109.22 109.675004) (width 0.3) (layer F.Cu) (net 21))
 (segment (start 109.22 109.675004) (end 109.219996 109.675) (width 0.3) (layer F.Cu) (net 21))
 (segment (start 110.000995 119.980999) (end 109.619999 119.600003) (width 0.3) (layer B.Cu) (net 21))
 (segment (start 120.194501 119.980999) (end 110.000995 119.980999) (width 0.3) (layer B.Cu) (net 21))
 (segment (start 121.71 118.4655) (end 120.194501 119.980999) (width 0.3) (layer B.Cu) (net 21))
 (segment (start 121.71 118.148) (end 121.71 118.4655) (width 0.3) (layer B.Cu) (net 21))
 (segment (start 109.619999 119.600003) (end 109.22 119.200004) (width 0.3) (layer B.Cu) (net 21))
 (via (at 109.22 119.200004) (size 0.8) (drill 0.4) (layers F.Cu B.Cu) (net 21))
 (segment (start 109.619995 109.275001) (end 109.219996 109.675) (width 0.3) (layer B.Cu) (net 21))
 (segment (start 110.28 108.614996) (end 109.619995 109.275001) (width 0.3) (layer B.Cu) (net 21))
 (via (at 109.219996 109.675) (size 0.8) (drill 0.4) (layers F.Cu B.Cu) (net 21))
 (segment (start 110.28 101.2) (end 110.28 108.614996) (width 0.3) (layer B.Cu) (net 21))
 (segment (start 81.6025 116.8505) (end 81.6025 108.0825) (width 0.3) (layer B.Cu) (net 1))
 (segment (start 81.6025 108.0825) (end 85.09 104.595) (width 0.3) (layer B.Cu) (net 1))
 (segment (start 85.09 104.595) (end 105.2195 104.595) (width 0.3) (layer B.Cu) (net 1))
 (segment (start 105.2195 104.595) (end 106.4895 105.865) (width 0.3) (layer B.Cu) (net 1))
 (segment (start 107.74 101.2) (end 107.74 104.6145) (width 0.3) (layer B.Cu) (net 1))
 (segment (start 107.74 104.6145) (end 106.4895 105.865) (width 0.3) (layer B.Cu) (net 1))
 (segment (start 107.74 101.2) (end 107.7595 101.2195) (width 0.3) (layer B.Cu) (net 1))
 (segment (start 120.44 118.148) (end 120.44 118.4655) (width 0.3) (layer B.Cu) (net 17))
 (segment (start 111.125 119.2) (end 109.22 117.295) (width 0.3) (layer B.Cu) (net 17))
 (segment (start 120.44 118.4655) (end 119.7055 119.2) (width 0.3) (layer B.Cu) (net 17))
 (segment (start 119.7055 119.2) (end 111.125 119.2) (width 0.3) (layer B.Cu) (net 17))
 (segment (start 109.22 117.295) (end 102.870012 117.295) (width 0.3) (layer B.Cu) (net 17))
 (segment (start 102.870012 117.295) (end 102.635011 117.530001) (width 0.3) (layer B.Cu) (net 17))
 (segment (start 102.635011 117.530001) (end 102.235012 117.93) (width 0.3) (layer B.Cu) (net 17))
 (segment (start 102.235012 117.93) (end 102.235012 110.310012) (width 0.3) (layer F.Cu) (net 17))
 (segment (start 102.235 117.929988) (end 102.235 110.31) (width 0.3) (layer F.Cu) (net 17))
 (segment (start 102.235 109.675) (end 102.235 110.31) (width 0.3) (layer B.Cu) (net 17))
 (segment (start 102.235012 110.310012) (end 102.235 110.31) (width 0.3) (layer F.Cu) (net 17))
 (via (at 102.235 110.31) (size 0.8) (drill 0.4) (layers F.Cu B.Cu) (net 17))
 (segment (start 102.235 105.5475) (end 102.235 109.675) (width 0.3) (layer B.Cu) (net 17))
 (via (at 102.235012 117.93) (size 0.8) (drill 0.4) (layers F.Cu B.Cu) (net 17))
 (segment (start 120.391 118.197) (end 120.44 118.148) (width 0.3) (layer B.Cu) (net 17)))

